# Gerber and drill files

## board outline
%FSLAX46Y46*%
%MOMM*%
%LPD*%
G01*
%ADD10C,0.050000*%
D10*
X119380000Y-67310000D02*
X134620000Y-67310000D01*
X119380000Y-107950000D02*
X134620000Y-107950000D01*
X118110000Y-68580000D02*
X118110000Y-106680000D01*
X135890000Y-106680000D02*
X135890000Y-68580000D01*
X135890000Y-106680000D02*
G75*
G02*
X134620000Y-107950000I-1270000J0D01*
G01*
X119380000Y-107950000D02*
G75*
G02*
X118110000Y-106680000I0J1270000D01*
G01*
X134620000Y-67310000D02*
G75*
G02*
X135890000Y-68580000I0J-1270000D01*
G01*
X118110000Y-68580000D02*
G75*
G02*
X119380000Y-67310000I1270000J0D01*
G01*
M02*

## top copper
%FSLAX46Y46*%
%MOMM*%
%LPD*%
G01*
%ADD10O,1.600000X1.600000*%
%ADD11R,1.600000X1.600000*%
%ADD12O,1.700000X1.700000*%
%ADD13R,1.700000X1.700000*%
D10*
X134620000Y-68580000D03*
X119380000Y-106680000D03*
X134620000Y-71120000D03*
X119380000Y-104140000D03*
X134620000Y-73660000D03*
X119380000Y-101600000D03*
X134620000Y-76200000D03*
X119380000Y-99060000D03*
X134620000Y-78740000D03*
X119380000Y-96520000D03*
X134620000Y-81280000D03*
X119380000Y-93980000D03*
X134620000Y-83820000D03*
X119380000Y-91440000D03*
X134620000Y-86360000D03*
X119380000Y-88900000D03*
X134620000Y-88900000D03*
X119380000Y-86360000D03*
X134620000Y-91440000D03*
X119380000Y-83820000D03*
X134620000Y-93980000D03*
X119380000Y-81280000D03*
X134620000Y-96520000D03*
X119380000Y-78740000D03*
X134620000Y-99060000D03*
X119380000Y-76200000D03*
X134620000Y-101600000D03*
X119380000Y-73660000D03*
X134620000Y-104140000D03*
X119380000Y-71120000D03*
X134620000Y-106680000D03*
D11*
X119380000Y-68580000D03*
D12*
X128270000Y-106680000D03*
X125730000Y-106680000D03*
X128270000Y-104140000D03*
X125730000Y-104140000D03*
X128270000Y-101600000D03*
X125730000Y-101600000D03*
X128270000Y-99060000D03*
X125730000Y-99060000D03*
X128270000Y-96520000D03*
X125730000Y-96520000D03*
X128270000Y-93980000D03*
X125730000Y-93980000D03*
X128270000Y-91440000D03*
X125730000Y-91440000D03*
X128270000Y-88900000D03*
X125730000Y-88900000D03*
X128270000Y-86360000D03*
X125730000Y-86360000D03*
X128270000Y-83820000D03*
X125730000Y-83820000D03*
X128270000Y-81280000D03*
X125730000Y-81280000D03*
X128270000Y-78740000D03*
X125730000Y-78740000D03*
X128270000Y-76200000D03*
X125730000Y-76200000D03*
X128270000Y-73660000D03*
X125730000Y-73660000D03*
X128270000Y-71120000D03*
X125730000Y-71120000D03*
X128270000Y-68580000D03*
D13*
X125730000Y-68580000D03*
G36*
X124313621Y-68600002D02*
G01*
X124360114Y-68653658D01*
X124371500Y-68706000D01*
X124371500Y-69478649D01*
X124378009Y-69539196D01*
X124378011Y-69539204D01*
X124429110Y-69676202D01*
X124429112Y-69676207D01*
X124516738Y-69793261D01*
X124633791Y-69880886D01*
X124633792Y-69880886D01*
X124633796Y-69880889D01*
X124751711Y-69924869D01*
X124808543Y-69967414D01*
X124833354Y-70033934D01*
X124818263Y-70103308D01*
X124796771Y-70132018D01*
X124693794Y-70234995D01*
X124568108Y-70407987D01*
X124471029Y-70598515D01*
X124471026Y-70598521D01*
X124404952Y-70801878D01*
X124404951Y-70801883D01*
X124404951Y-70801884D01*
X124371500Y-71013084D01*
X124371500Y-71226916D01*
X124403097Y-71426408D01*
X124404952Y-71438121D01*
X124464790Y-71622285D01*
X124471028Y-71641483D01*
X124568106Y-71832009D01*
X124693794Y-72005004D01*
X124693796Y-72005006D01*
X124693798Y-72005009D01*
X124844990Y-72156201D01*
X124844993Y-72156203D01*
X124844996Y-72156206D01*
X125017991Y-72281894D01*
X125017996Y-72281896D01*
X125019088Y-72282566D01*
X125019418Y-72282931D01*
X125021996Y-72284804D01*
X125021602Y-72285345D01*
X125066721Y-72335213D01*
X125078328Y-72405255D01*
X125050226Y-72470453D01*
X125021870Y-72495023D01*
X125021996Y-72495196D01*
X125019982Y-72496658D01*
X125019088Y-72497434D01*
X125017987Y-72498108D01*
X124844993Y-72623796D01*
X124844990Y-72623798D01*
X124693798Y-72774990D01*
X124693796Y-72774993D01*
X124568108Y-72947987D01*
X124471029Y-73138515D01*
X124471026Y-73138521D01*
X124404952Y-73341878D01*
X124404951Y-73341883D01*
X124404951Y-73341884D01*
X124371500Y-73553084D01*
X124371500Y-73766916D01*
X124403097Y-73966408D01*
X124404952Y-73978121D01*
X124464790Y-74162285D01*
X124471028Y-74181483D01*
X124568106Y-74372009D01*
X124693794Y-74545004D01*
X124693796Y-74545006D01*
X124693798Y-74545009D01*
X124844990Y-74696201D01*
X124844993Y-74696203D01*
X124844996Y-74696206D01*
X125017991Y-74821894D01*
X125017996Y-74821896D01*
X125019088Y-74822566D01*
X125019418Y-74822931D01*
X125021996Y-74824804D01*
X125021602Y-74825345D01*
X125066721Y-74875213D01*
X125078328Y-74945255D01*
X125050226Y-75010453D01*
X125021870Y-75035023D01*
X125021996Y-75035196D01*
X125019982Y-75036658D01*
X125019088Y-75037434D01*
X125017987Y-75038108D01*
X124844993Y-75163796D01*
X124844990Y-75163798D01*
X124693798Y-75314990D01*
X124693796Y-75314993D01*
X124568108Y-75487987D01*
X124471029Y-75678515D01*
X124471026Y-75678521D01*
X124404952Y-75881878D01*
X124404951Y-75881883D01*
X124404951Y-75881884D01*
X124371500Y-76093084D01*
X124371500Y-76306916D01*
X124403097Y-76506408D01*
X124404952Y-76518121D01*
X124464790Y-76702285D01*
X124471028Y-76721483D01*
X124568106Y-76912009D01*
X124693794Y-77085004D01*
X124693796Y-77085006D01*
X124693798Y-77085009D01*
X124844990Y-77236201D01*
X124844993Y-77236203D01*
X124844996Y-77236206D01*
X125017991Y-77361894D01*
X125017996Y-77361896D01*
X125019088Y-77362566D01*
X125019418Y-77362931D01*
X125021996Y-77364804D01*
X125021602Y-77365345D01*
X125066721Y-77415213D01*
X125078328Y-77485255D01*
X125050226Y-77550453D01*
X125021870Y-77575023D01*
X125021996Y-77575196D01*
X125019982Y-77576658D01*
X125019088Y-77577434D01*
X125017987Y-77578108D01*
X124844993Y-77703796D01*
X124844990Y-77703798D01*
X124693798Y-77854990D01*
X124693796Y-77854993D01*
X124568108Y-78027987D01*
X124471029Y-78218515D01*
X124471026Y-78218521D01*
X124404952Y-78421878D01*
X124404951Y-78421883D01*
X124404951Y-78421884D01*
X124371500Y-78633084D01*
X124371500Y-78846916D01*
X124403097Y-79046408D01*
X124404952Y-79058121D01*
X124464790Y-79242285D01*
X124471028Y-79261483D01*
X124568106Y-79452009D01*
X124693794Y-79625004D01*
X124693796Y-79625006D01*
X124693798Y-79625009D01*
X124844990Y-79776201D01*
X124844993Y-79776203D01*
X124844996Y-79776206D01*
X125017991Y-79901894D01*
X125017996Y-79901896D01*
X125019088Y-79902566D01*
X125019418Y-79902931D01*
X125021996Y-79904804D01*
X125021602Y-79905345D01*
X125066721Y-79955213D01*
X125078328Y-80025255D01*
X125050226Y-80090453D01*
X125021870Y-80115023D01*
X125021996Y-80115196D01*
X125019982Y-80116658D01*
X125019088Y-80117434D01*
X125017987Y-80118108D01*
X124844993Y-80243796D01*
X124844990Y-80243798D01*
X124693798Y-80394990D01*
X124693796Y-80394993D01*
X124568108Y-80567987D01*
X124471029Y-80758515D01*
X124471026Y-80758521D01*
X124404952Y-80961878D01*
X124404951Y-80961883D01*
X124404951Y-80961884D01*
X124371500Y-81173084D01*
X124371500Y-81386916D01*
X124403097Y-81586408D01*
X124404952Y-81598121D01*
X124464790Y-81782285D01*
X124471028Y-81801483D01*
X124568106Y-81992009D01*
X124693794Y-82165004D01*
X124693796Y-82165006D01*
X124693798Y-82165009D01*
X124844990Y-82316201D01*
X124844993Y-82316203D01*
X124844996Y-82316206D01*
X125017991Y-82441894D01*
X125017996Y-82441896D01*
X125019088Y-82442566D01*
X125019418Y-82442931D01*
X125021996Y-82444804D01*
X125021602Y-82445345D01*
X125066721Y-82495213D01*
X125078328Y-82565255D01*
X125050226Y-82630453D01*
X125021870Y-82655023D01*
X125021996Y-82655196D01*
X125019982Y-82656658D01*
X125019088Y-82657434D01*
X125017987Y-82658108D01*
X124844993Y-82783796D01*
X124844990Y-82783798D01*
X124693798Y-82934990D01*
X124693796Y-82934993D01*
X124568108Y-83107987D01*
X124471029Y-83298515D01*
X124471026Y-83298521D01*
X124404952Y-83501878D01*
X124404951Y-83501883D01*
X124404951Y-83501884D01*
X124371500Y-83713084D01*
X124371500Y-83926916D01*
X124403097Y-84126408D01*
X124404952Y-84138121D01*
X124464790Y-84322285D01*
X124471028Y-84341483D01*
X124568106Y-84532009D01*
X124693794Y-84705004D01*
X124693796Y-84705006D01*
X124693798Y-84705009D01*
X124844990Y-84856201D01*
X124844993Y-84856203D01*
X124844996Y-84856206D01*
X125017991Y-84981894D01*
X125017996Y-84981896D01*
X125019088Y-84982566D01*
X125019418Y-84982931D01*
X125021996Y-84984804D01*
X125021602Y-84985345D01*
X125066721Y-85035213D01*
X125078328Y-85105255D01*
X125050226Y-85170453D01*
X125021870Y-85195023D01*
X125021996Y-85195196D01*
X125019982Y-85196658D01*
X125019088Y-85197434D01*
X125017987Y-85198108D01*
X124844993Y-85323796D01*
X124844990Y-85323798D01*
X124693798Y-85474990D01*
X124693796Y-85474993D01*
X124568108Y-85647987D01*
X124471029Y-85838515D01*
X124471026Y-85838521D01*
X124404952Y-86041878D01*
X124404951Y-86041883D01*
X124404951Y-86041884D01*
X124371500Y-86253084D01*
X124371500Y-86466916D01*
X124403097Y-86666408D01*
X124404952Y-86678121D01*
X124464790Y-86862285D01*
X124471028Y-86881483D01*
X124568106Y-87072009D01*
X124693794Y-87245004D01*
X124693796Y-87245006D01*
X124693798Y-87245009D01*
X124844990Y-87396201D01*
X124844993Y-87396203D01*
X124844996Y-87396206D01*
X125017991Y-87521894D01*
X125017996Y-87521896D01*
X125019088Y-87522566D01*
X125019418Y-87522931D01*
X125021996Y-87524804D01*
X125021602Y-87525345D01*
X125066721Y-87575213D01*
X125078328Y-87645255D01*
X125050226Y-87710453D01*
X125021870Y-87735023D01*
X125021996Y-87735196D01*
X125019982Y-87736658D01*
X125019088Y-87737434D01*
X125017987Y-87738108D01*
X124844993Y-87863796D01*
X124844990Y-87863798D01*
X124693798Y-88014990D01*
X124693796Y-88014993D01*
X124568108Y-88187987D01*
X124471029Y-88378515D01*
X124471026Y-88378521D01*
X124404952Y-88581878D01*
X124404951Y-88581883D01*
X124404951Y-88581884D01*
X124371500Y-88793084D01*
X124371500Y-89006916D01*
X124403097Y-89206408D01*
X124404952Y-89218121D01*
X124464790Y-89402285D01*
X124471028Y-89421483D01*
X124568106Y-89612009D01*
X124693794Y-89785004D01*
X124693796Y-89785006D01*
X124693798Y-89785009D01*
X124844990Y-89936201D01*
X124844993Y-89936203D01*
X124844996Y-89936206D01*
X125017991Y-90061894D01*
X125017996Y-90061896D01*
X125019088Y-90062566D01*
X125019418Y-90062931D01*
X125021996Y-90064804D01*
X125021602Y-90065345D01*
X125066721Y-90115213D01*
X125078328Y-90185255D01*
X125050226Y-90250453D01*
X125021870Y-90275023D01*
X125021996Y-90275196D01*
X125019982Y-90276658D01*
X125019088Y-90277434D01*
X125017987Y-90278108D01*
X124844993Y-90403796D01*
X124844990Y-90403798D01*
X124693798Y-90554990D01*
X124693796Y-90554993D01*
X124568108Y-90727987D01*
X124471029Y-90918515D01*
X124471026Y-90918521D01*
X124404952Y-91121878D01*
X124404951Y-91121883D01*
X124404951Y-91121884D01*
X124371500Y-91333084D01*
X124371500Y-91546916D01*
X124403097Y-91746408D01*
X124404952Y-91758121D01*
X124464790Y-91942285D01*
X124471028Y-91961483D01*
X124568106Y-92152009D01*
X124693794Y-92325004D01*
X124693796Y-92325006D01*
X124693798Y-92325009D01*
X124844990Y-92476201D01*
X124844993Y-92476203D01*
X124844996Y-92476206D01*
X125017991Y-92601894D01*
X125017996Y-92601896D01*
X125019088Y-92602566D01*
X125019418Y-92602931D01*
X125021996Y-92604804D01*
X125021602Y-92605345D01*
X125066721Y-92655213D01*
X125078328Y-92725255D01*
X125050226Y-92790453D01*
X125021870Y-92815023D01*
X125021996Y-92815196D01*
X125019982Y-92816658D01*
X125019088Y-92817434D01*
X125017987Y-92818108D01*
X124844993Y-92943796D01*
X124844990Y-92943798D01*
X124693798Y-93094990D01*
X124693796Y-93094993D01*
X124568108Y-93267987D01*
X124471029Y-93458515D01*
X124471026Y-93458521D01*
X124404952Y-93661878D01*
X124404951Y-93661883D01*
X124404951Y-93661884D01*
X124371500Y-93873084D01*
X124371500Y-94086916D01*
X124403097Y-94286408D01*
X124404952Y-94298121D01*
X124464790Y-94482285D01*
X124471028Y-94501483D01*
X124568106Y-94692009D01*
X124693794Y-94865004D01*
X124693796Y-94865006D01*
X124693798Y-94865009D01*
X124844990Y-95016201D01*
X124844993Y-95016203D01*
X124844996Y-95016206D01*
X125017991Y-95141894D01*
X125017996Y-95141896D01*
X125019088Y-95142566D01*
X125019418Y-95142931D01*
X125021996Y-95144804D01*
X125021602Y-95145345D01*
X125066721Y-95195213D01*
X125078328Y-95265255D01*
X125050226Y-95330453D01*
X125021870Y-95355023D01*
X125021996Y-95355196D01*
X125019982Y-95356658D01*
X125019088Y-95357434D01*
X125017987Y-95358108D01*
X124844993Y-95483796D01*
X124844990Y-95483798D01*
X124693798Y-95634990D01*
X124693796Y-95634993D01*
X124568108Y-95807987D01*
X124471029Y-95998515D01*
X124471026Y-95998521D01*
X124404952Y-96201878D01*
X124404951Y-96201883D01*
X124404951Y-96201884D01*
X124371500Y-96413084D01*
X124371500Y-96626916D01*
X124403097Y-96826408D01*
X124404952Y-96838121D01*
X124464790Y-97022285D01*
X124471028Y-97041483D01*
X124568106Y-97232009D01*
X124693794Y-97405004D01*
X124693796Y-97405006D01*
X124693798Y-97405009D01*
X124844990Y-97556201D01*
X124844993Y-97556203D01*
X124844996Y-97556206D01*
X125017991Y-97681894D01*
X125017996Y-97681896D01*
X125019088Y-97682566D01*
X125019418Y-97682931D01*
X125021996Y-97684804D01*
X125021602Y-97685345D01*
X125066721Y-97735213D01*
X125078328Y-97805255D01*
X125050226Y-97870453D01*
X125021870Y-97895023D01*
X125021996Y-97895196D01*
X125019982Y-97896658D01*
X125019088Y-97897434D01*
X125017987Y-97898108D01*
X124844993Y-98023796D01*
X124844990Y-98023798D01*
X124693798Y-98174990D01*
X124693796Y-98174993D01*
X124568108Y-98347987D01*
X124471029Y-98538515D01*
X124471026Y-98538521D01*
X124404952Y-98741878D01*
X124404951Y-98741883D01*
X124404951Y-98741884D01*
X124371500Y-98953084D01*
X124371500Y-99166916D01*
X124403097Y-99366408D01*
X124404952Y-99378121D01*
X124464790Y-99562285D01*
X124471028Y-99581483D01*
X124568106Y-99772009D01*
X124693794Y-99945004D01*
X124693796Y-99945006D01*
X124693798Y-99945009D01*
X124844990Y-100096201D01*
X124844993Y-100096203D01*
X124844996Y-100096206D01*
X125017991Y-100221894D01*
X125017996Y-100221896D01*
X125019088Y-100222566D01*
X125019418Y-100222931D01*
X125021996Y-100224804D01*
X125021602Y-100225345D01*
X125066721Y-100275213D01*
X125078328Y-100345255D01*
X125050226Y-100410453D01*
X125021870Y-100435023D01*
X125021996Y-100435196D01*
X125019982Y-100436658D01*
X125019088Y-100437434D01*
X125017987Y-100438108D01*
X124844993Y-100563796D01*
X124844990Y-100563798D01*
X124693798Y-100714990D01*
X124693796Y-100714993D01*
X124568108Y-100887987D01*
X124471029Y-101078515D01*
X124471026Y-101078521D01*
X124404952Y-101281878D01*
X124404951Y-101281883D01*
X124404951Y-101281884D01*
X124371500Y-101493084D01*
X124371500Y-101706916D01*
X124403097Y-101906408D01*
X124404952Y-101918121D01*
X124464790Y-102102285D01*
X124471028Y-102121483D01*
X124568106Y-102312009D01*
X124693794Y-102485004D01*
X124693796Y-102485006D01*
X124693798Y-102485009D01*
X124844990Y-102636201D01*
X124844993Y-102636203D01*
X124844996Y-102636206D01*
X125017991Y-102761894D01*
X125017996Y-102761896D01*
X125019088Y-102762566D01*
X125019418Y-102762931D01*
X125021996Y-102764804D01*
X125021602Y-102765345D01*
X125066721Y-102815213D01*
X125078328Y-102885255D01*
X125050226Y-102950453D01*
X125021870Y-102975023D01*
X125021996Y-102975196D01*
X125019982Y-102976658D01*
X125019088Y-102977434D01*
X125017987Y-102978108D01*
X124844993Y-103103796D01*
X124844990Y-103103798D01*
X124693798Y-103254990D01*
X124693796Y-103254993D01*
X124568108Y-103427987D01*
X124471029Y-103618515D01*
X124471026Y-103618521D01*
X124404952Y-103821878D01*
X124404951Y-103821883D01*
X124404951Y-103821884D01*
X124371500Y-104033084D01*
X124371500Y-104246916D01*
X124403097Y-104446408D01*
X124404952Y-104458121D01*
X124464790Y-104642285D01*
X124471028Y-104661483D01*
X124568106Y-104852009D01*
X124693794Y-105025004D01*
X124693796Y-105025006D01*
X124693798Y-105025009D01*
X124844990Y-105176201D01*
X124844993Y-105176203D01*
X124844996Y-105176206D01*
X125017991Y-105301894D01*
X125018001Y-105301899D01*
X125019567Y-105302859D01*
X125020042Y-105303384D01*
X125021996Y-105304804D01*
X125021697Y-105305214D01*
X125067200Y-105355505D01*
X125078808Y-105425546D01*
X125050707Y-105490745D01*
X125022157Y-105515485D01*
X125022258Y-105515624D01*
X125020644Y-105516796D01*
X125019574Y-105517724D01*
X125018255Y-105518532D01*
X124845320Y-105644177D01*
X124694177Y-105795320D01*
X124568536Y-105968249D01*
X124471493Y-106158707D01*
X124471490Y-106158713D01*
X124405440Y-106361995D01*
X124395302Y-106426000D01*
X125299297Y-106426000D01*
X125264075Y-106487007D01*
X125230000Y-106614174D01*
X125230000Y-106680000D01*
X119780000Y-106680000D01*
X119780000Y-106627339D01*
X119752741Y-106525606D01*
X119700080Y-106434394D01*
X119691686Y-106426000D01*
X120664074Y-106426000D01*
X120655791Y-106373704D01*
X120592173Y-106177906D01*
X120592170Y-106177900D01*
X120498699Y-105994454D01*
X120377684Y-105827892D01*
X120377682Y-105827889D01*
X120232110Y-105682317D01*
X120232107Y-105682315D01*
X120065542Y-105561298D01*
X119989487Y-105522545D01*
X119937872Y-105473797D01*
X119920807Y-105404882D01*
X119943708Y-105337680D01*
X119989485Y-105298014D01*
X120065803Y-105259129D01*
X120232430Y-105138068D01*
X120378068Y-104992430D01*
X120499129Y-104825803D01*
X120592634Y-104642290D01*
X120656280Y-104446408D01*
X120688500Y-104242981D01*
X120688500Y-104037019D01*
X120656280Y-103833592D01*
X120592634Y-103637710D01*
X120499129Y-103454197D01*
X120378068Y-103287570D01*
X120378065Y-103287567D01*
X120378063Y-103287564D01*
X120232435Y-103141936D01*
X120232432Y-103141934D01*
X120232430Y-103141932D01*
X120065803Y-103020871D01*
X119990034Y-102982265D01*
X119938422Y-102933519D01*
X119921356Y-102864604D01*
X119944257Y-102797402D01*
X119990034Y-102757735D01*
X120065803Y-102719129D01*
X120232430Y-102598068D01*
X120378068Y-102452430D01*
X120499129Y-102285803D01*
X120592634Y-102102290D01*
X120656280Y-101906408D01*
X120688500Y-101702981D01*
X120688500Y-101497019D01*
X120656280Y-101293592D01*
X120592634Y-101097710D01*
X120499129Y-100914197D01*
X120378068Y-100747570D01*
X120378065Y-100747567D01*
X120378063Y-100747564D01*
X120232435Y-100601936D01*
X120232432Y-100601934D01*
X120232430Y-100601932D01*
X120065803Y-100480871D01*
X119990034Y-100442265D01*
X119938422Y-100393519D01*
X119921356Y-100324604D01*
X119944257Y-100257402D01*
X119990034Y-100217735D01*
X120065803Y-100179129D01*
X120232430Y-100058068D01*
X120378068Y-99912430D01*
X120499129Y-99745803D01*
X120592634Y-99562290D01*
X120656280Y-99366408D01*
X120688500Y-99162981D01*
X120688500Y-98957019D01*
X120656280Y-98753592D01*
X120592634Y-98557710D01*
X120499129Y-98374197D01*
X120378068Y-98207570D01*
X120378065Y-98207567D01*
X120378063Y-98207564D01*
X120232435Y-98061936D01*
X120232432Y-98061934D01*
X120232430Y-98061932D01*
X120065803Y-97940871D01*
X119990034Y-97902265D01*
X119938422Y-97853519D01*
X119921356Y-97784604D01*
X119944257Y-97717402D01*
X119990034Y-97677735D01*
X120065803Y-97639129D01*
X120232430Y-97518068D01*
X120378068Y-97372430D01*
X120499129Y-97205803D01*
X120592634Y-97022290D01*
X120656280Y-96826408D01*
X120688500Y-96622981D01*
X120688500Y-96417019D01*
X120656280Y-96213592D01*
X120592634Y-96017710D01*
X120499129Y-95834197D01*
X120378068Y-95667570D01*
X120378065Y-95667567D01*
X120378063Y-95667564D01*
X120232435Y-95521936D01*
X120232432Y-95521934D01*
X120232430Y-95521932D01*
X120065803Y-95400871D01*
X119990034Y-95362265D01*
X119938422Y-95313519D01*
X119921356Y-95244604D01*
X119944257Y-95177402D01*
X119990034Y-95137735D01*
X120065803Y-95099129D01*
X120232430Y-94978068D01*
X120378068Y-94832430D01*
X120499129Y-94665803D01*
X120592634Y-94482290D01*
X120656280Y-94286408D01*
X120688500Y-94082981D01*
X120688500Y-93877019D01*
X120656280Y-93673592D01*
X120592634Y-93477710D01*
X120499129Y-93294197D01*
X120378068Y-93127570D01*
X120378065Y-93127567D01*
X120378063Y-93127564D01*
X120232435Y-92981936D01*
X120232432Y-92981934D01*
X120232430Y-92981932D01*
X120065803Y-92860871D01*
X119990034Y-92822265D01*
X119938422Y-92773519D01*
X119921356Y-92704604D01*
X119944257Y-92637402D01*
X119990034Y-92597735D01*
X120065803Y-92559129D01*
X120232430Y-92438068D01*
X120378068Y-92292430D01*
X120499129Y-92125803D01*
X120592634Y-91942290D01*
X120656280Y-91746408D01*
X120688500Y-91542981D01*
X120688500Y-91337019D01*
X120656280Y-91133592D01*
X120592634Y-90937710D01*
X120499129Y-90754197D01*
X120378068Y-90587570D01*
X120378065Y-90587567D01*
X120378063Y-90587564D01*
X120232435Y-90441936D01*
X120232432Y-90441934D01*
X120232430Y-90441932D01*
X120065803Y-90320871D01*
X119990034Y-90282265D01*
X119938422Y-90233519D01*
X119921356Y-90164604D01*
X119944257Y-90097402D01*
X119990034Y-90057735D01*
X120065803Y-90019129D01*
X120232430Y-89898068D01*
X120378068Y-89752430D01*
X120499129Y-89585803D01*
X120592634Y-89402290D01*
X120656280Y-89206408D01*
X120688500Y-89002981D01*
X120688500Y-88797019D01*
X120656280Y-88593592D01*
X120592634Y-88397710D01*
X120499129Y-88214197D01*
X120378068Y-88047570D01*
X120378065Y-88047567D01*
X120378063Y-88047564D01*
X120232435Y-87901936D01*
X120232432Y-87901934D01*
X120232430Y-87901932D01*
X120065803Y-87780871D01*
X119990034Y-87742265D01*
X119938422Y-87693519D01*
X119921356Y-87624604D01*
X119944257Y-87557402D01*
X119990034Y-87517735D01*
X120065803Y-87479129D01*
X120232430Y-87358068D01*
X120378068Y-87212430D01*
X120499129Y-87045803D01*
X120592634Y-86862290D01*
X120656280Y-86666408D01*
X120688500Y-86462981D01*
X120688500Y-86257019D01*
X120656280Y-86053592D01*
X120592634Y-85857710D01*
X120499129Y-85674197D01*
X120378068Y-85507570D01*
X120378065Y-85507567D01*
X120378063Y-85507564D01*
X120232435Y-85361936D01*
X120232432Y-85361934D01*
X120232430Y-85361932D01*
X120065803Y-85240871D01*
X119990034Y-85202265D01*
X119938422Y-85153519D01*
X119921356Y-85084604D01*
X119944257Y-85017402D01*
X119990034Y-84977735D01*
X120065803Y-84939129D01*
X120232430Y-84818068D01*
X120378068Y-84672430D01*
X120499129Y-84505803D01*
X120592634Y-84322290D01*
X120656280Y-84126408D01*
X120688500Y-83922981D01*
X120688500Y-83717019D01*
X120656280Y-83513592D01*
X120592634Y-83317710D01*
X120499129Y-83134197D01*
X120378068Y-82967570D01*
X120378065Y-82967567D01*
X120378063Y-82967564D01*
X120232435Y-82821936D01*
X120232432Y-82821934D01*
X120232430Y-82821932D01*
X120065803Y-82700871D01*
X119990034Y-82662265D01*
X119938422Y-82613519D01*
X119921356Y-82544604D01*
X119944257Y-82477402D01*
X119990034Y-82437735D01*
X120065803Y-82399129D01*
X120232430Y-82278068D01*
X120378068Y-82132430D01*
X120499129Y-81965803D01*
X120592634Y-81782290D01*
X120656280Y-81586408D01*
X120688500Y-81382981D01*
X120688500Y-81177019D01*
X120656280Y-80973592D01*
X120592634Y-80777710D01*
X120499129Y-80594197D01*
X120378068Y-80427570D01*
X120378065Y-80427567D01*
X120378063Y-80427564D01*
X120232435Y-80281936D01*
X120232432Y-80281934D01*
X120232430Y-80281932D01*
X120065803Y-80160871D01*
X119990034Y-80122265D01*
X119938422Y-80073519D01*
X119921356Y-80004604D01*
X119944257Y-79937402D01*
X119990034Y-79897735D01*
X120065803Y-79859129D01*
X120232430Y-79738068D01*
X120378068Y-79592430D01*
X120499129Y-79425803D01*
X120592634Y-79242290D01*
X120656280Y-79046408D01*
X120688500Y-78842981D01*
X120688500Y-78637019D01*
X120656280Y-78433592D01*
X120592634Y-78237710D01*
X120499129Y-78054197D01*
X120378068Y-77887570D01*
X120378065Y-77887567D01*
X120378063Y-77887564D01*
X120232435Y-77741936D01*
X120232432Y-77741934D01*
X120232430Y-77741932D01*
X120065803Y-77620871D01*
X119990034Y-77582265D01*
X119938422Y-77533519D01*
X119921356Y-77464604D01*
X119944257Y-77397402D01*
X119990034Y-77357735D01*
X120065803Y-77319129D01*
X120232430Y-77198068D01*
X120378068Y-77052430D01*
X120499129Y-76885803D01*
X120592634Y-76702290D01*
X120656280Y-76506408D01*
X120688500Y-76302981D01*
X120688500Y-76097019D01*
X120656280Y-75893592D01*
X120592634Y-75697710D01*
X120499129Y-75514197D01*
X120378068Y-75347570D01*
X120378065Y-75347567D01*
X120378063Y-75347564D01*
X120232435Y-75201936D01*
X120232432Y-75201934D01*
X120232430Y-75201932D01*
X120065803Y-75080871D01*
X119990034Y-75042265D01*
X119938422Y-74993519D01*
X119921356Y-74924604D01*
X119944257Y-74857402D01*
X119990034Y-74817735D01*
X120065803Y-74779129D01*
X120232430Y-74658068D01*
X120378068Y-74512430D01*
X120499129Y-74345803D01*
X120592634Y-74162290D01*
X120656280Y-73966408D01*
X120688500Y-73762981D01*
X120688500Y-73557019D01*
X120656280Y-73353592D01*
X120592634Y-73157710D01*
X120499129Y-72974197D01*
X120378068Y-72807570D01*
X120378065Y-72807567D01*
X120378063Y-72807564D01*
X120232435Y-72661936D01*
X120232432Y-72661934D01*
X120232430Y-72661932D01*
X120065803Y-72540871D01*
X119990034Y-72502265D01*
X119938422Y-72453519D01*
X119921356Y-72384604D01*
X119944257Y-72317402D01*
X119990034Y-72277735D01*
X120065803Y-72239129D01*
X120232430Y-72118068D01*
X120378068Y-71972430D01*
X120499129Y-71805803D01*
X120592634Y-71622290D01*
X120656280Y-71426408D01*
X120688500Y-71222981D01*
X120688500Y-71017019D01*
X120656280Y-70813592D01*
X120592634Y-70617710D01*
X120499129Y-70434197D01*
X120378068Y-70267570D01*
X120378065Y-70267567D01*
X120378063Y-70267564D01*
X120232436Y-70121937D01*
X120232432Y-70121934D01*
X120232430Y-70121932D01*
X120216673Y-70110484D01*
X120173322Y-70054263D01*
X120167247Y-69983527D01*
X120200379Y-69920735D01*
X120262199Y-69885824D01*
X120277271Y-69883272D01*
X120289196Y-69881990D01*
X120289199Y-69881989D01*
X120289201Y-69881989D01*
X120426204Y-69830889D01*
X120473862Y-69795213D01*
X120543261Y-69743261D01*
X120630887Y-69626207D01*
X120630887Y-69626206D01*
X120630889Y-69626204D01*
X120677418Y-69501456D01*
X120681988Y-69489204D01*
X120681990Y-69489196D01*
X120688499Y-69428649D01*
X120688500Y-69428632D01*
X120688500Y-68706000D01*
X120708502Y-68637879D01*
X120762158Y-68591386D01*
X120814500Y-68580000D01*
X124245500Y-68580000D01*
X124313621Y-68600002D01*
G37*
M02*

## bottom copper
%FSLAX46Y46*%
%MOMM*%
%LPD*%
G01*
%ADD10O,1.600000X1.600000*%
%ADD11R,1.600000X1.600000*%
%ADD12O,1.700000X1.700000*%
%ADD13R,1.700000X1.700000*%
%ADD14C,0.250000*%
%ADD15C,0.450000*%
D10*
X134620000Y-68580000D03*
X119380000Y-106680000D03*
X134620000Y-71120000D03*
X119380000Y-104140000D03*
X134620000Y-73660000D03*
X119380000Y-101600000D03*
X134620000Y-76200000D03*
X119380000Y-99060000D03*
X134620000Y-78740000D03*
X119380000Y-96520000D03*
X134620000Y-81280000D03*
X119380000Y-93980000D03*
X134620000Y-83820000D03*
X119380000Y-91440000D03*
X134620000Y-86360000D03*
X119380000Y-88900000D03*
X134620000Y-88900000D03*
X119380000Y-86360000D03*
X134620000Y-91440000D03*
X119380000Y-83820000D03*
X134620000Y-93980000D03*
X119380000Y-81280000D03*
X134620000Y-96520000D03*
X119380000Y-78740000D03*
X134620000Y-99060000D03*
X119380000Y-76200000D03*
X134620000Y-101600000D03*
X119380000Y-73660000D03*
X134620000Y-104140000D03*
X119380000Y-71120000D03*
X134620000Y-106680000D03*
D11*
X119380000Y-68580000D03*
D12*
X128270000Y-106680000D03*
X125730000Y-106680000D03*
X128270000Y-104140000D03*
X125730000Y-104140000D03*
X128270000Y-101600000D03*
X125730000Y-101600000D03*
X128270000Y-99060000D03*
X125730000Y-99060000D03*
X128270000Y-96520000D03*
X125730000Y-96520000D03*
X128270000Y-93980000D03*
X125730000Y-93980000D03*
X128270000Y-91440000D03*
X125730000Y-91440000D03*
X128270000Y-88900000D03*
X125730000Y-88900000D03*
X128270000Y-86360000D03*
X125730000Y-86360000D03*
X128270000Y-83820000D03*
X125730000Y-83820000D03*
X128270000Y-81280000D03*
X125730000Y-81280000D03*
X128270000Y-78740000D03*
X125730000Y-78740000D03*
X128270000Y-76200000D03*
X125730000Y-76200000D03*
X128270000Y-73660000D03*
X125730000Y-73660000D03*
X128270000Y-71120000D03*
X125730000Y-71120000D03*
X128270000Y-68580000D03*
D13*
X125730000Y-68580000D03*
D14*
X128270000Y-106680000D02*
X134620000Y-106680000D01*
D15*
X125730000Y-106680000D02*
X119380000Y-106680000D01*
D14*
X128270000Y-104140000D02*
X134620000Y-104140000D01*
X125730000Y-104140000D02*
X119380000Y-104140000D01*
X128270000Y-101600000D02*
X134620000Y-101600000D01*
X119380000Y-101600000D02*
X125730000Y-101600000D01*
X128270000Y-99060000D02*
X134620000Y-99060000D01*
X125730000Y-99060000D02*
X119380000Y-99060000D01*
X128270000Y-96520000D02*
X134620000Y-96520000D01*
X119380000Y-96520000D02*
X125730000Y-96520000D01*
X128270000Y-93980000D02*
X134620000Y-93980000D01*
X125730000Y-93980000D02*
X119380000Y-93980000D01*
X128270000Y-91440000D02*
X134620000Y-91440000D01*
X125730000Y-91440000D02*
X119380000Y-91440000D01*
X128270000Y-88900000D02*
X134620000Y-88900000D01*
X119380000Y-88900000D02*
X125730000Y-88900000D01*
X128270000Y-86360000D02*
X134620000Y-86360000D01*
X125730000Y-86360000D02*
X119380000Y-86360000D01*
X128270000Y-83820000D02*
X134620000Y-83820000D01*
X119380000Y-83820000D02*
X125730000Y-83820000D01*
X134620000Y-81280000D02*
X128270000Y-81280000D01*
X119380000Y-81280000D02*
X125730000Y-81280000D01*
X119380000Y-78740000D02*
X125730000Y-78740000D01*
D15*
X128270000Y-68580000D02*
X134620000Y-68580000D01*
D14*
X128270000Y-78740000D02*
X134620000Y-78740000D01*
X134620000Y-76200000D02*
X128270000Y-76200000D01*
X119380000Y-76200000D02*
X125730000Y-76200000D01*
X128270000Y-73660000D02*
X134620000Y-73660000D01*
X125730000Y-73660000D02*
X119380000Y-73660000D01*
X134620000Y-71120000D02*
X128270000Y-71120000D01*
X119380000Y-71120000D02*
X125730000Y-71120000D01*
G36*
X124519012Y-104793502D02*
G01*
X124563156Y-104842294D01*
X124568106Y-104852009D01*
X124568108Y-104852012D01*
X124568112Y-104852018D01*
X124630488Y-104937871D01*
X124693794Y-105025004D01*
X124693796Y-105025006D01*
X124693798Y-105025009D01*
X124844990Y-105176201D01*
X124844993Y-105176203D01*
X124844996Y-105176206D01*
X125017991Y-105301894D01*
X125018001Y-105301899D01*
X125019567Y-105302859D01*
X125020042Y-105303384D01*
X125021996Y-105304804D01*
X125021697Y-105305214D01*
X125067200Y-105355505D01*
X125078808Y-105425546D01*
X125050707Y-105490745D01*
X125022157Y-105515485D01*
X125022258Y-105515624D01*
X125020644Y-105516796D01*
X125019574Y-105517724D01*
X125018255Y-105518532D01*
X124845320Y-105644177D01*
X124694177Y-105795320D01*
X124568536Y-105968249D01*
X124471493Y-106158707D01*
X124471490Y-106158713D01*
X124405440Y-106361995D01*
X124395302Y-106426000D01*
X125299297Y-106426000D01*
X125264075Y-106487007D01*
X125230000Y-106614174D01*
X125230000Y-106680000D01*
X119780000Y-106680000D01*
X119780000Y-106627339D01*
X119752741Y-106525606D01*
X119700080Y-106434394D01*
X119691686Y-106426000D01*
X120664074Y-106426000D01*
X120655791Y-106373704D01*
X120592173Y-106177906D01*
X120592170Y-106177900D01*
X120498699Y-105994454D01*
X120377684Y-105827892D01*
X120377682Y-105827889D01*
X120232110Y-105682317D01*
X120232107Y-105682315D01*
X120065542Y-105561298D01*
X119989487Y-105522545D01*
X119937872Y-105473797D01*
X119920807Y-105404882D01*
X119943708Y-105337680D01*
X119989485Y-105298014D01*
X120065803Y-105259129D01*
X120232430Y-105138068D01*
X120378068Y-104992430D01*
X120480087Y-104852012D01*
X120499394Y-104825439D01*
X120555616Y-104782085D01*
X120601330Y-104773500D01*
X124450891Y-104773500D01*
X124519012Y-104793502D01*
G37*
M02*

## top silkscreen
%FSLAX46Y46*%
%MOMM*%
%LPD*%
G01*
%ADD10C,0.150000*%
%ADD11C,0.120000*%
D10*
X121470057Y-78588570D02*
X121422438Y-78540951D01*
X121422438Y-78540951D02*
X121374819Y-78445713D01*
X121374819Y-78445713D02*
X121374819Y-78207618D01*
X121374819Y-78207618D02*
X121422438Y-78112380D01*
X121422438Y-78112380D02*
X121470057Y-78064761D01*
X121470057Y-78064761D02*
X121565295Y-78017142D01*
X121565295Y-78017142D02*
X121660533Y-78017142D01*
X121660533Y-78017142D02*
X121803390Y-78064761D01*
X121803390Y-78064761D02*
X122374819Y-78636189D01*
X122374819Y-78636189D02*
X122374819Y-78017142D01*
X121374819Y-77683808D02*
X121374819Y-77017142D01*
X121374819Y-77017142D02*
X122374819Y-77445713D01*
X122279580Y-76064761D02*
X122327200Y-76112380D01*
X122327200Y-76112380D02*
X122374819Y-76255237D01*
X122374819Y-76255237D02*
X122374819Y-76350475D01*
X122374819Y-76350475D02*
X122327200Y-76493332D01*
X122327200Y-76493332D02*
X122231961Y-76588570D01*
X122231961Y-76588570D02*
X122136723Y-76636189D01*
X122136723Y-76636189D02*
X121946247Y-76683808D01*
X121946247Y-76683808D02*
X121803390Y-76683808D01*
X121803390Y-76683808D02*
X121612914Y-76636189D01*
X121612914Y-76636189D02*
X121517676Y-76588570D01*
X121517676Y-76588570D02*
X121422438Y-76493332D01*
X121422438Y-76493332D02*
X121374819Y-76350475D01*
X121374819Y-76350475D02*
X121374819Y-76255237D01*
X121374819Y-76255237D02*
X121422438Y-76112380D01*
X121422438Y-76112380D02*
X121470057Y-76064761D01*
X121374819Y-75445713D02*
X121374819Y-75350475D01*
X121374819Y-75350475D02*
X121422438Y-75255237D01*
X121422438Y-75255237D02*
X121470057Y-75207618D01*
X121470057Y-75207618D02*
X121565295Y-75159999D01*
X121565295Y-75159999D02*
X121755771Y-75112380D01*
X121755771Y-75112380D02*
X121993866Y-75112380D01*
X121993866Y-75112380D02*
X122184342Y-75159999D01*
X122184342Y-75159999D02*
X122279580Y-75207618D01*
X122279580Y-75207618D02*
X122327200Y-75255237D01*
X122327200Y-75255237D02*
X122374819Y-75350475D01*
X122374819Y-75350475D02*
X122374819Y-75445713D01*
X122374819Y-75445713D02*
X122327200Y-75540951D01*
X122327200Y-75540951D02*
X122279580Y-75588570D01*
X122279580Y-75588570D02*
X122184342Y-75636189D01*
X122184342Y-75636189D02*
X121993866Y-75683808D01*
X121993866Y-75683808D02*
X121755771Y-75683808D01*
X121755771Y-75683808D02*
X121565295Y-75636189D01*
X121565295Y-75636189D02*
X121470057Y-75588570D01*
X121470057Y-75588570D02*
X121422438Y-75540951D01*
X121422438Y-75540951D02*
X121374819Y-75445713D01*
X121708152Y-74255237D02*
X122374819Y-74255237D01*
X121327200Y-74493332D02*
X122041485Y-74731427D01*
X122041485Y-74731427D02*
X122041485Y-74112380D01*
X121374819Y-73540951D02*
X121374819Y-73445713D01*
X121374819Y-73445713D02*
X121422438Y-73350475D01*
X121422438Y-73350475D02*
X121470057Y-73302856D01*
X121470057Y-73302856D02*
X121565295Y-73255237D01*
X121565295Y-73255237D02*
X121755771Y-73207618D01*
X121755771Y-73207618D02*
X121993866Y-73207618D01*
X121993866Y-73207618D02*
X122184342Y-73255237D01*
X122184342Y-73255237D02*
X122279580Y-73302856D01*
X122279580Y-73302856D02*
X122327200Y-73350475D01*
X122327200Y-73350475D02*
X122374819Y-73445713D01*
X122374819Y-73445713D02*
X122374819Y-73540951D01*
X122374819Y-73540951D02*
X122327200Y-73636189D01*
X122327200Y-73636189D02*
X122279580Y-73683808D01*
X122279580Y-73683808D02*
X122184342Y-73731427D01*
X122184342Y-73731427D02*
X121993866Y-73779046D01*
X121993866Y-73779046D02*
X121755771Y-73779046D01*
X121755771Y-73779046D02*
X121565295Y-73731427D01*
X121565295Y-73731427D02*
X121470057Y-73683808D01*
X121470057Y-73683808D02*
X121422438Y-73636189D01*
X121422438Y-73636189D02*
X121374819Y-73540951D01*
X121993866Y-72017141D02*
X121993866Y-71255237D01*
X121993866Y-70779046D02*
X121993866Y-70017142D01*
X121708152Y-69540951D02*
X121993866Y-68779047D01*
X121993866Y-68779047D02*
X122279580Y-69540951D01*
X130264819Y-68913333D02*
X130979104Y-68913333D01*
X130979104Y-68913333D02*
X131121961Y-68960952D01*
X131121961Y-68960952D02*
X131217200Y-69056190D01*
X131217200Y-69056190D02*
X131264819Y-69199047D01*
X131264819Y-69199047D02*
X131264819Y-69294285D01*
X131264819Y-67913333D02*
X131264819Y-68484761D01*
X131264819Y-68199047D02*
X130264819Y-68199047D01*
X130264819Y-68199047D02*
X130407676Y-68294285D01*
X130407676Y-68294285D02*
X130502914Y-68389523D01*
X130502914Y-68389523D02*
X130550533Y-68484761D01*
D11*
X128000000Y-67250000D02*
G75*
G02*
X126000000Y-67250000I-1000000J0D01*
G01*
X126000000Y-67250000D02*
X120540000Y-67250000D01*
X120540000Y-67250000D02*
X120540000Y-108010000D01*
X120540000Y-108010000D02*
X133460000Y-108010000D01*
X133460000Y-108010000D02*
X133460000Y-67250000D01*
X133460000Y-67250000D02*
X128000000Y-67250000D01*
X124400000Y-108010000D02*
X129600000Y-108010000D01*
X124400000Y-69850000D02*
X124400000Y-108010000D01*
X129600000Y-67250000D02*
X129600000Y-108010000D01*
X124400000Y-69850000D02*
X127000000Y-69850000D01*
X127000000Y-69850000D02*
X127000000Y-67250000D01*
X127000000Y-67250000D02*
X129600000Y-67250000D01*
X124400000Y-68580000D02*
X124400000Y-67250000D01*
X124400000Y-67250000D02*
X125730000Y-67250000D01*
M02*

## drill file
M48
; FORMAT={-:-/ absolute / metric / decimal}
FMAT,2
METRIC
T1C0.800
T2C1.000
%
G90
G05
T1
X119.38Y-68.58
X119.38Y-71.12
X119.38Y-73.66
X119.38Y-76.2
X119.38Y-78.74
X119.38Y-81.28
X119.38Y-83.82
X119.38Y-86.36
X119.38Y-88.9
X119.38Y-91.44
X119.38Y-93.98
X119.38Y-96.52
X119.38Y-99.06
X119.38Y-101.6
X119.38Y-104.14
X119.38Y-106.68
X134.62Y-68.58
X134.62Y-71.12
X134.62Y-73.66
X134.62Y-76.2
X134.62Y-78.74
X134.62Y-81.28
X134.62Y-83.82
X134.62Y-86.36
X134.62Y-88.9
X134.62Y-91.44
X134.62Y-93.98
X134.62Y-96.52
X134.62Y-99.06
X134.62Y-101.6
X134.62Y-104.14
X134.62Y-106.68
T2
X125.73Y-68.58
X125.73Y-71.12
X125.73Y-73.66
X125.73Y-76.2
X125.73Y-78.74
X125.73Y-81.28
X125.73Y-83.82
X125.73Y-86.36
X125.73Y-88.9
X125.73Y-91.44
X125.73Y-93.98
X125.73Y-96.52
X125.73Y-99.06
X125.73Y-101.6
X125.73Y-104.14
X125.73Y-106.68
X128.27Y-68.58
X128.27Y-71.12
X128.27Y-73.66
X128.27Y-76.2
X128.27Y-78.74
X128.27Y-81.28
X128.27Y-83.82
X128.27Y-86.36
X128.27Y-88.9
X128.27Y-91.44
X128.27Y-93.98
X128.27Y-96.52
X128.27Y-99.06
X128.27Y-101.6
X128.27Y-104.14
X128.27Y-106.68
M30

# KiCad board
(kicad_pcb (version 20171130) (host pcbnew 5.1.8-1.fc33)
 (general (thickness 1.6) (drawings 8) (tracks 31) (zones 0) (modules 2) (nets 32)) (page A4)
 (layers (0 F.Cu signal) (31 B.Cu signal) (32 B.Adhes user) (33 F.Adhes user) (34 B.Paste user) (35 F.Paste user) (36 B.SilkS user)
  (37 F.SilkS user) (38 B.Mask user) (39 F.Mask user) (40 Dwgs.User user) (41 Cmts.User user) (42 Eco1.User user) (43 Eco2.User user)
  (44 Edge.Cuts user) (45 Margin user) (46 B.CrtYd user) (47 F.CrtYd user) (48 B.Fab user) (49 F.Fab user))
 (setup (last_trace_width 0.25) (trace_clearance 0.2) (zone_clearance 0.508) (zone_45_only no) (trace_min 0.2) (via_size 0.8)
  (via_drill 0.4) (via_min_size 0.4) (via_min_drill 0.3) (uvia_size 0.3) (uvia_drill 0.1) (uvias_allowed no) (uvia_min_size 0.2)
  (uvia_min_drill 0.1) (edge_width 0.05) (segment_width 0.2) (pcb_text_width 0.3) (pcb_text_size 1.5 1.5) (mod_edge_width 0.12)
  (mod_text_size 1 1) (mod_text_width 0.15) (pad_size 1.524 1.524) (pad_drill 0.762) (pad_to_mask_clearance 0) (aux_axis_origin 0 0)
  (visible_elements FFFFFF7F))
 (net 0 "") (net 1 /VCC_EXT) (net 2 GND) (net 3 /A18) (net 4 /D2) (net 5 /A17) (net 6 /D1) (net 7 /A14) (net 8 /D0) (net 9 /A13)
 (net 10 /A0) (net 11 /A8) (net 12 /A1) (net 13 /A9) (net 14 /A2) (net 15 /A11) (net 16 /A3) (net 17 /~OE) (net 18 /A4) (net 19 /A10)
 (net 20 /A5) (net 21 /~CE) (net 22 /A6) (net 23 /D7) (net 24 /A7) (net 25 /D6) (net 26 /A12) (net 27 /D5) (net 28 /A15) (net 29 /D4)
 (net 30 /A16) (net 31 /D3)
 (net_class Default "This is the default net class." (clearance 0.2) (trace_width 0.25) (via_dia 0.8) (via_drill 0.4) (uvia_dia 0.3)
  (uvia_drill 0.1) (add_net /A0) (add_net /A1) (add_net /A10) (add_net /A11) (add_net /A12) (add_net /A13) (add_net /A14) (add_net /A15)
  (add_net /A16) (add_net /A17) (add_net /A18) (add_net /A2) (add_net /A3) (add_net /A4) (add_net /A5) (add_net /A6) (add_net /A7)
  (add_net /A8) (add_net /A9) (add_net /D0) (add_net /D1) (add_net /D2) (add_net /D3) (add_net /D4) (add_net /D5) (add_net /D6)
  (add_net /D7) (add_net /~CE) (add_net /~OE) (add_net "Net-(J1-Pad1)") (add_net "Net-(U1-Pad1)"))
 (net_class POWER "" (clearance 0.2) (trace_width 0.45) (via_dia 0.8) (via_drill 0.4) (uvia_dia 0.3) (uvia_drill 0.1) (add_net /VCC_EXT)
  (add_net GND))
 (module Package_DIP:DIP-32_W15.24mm (layer F.Cu) (at 119.38 68.58)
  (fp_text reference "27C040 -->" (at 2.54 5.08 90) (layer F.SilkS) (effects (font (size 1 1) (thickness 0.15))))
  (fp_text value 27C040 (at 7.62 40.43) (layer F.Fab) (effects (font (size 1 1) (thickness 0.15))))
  (fp_arc (start 7.62 -1.33) (end 6.62 -1.33) (angle -180) (layer F.SilkS) (width 0.12))
  (fp_line (start 6.62 -1.33) (end 1.16 -1.33) (layer F.SilkS) (width 0.12))
  (fp_line (start 1.16 -1.33) (end 1.16 39.43) (layer F.SilkS) (width 0.12))
  (fp_line (start 1.16 39.43) (end 14.08 39.43) (layer F.SilkS) (width 0.12))
  (fp_line (start 14.08 39.43) (end 14.08 -1.33) (layer F.SilkS) (width 0.12))
  (fp_line (start 14.08 -1.33) (end 8.62 -1.33) (layer F.SilkS) (width 0.12))
  (pad 32 thru_hole oval (at 15.24 0) (size 1.6 1.6) (drill 0.8) (layers *.Cu *.Mask) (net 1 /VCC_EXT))
  (pad 16 thru_hole oval (at 0 38.1) (size 1.6 1.6) (drill 0.8) (layers *.Cu *.Mask) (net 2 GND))
  (pad 31 thru_hole oval (at 15.24 2.54) (size 1.6 1.6) (drill 0.8) (layers *.Cu *.Mask) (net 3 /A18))
  (pad 15 thru_hole oval (at 0 35.56) (size 1.6 1.6) (drill 0.8) (layers *.Cu *.Mask) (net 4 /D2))
  (pad 30 thru_hole oval (at 15.24 5.08) (size 1.6 1.6) (drill 0.8) (layers *.Cu *.Mask) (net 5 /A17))
  (pad 14 thru_hole oval (at 0 33.02) (size 1.6 1.6) (drill 0.8) (layers *.Cu *.Mask) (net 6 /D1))
  (pad 29 thru_hole oval (at 15.24 7.62) (size 1.6 1.6) (drill 0.8) (layers *.Cu *.Mask) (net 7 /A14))
  (pad 13 thru_hole oval (at 0 30.48) (size 1.6 1.6) (drill 0.8) (layers *.Cu *.Mask) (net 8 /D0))
  (pad 28 thru_hole oval (at 15.24 10.16) (size 1.6 1.6) (drill 0.8) (layers *.Cu *.Mask) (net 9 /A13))
  (pad 12 thru_hole oval (at 0 27.94) (size 1.6 1.6) (drill 0.8) (layers *.Cu *.Mask) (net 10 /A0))
  (pad 27 thru_hole oval (at 15.24 12.7) (size 1.6 1.6) (drill 0.8) (layers *.Cu *.Mask) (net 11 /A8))
  (pad 11 thru_hole oval (at 0 25.4) (size 1.6 1.6) (drill 0.8) (layers *.Cu *.Mask) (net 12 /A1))
  (pad 26 thru_hole oval (at 15.24 15.24) (size 1.6 1.6) (drill 0.8) (layers *.Cu *.Mask) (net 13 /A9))
  (pad 10 thru_hole oval (at 0 22.86) (size 1.6 1.6) (drill 0.8) (layers *.Cu *.Mask) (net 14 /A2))
  (pad 25 thru_hole oval (at 15.24 17.78) (size 1.6 1.6) (drill 0.8) (layers *.Cu *.Mask) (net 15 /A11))
  (pad 9 thru_hole oval (at 0 20.32) (size 1.6 1.6) (drill 0.8) (layers *.Cu *.Mask) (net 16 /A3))
  (pad 24 thru_hole oval (at 15.24 20.32) (size 1.6 1.6) (drill 0.8) (layers *.Cu *.Mask) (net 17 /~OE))
  (pad 8 thru_hole oval (at 0 17.78) (size 1.6 1.6) (drill 0.8) (layers *.Cu *.Mask) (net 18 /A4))
  (pad 23 thru_hole oval (at 15.24 22.86) (size 1.6 1.6) (drill 0.8) (layers *.Cu *.Mask) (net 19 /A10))
  (pad 7 thru_hole oval (at 0 15.24) (size 1.6 1.6) (drill 0.8) (layers *.Cu *.Mask) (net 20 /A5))
  (pad 22 thru_hole oval (at 15.24 25.4) (size 1.6 1.6) (drill 0.8) (layers *.Cu *.Mask) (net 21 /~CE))
  (pad 6 thru_hole oval (at 0 12.7) (size 1.6 1.6) (drill 0.8) (layers *.Cu *.Mask) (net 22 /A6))
  (pad 21 thru_hole oval (at 15.24 27.94) (size 1.6 1.6) (drill 0.8) (layers *.Cu *.Mask) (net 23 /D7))
  (pad 5 thru_hole oval (at 0 10.16) (size 1.6 1.6) (drill 0.8) (layers *.Cu *.Mask) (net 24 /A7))
  (pad 20 thru_hole oval (at 15.24 30.48) (size 1.6 1.6) (drill 0.8) (layers *.Cu *.Mask) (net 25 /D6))
  (pad 4 thru_hole oval (at 0 7.62) (size 1.6 1.6) (drill 0.8) (layers *.Cu *.Mask) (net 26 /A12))
  (pad 19 thru_hole oval (at 15.24 33.02) (size 1.6 1.6) (drill 0.8) (layers *.Cu *.Mask) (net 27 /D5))
  (pad 3 thru_hole oval (at 0 5.08) (size 1.6 1.6) (drill 0.8) (layers *.Cu *.Mask) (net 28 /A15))
  (pad 18 thru_hole oval (at 15.24 35.56) (size 1.6 1.6) (drill 0.8) (layers *.Cu *.Mask) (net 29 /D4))
  (pad 2 thru_hole oval (at 0 2.54) (size 1.6 1.6) (drill 0.8) (layers *.Cu *.Mask) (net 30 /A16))
  (pad 17 thru_hole oval (at 15.24 38.1) (size 1.6 1.6) (drill 0.8) (layers *.Cu *.Mask) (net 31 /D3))
  (pad 1 thru_hole rect (at 0 0) (size 1.6 1.6) (drill 0.8) (layers *.Cu *.Mask)))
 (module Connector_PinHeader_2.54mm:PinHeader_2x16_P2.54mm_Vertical (layer F.Cu) (at 125.73 68.58)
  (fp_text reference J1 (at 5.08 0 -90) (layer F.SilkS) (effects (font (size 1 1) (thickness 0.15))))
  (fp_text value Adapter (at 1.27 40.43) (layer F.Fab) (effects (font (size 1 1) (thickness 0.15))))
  (fp_line (start -1.33 39.43) (end 3.87 39.43) (layer F.SilkS) (width 0.12))
  (fp_line (start -1.33 1.27) (end -1.33 39.43) (layer F.SilkS) (width 0.12))
  (fp_line (start 3.87 -1.33) (end 3.87 39.43) (layer F.SilkS) (width 0.12))
  (fp_line (start -1.33 1.27) (end 1.27 1.27) (layer F.SilkS) (width 0.12))
  (fp_line (start 1.27 1.27) (end 1.27 -1.33) (layer F.SilkS) (width 0.12))
  (fp_line (start 1.27 -1.33) (end 3.87 -1.33) (layer F.SilkS) (width 0.12))
  (fp_line (start -1.33 0) (end -1.33 -1.33) (layer F.SilkS) (width 0.12))
  (fp_line (start -1.33 -1.33) (end 0 -1.33) (layer F.SilkS) (width 0.12))
  (pad 32 thru_hole oval (at 2.54 38.1) (size 1.7 1.7) (drill 1) (layers *.Cu *.Mask) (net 31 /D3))
  (pad 31 thru_hole oval (at 0 38.1) (size 1.7 1.7) (drill 1) (layers *.Cu *.Mask) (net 2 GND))
  (pad 30 thru_hole oval (at 2.54 35.56) (size 1.7 1.7) (drill 1) (layers *.Cu *.Mask) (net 29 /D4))
  (pad 29 thru_hole oval (at 0 35.56) (size 1.7 1.7) (drill 1) (layers *.Cu *.Mask) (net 4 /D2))
  (pad 28 thru_hole oval (at 2.54 33.02) (size 1.7 1.7) (drill 1) (layers *.Cu *.Mask) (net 27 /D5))
  (pad 27 thru_hole oval (at 0 33.02) (size 1.7 1.7) (drill 1) (layers *.Cu *.Mask) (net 6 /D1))
  (pad 26 thru_hole oval (at 2.54 30.48) (size 1.7 1.7) (drill 1) (layers *.Cu *.Mask) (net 25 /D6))
  (pad 25 thru_hole oval (at 0 30.48) (size 1.7 1.7) (drill 1) (layers *.Cu *.Mask) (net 8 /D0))
  (pad 24 thru_hole oval (at 2.54 27.94) (size 1.7 1.7) (drill 1) (layers *.Cu *.Mask) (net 23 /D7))
  (pad 23 thru_hole oval (at 0 27.94) (size 1.7 1.7) (drill 1) (layers *.Cu *.Mask) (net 10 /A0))
  (pad 22 thru_hole oval (at 2.54 25.4) (size 1.7 1.7) (drill 1) (layers *.Cu *.Mask) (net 21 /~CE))
  (pad 21 thru_hole oval (at 0 25.4) (size 1.7 1.7) (drill 1) (layers *.Cu *.Mask) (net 12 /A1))
  (pad 20 thru_hole oval (at 2.54 22.86) (size 1.7 1.7) (drill 1) (layers *.Cu *.Mask) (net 19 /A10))
  (pad 19 thru_hole oval (at 0 22.86) (size 1.7 1.7) (drill 1) (layers *.Cu *.Mask) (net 14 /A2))
  (pad 18 thru_hole oval (at 2.54 20.32) (size 1.7 1.7) (drill 1) (layers *.Cu *.Mask) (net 17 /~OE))
  (pad 17 thru_hole oval (at 0 20.32) (size 1.7 1.7) (drill 1) (layers *.Cu *.Mask) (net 16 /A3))
  (pad 16 thru_hole oval (at 2.54 17.78) (size 1.7 1.7) (drill 1) (layers *.Cu *.Mask) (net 15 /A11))
  (pad 15 thru_hole oval (at 0 17.78) (size 1.7 1.7) (drill 1) (layers *.Cu *.Mask) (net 18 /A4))
  (pad 14 thru_hole oval (at 2.54 15.24) (size 1.7 1.7) (drill 1) (layers *.Cu *.Mask) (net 13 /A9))
  (pad 13 thru_hole oval (at 0 15.24) (size 1.7 1.7) (drill 1) (layers *.Cu *.Mask) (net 20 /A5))
  (pad 12 thru_hole oval (at 2.54 12.7) (size 1.7 1.7) (drill 1) (layers *.Cu *.Mask) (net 11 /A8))
  (pad 11 thru_hole oval (at 0 12.7) (size 1.7 1.7) (drill 1) (layers *.Cu *.Mask) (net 22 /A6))
  (pad 10 thru_hole oval (at 2.54 10.16) (size 1.7 1.7) (drill 1) (layers *.Cu *.Mask) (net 9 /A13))
  (pad 9 thru_hole oval (at 0 10.16) (size 1.7 1.7) (drill 1) (layers *.Cu *.Mask) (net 24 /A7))
  (pad 8 thru_hole oval (at 2.54 7.62) (size 1.7 1.7) (drill 1) (layers *.Cu *.Mask) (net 7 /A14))
  (pad 7 thru_hole oval (at 0 7.62) (size 1.7 1.7) (drill 1) (layers *.Cu *.Mask) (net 26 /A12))
  (pad 6 thru_hole oval (at 2.54 5.08) (size 1.7 1.7) (drill 1) (layers *.Cu *.Mask) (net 5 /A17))
  (pad 5 thru_hole oval (at 0 5.08) (size 1.7 1.7) (drill 1) (layers *.Cu *.Mask) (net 28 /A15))
  (pad 4 thru_hole oval (at 2.54 2.54) (size 1.7 1.7) (drill 1) (layers *.Cu *.Mask) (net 3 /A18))
  (pad 3 thru_hole oval (at 0 2.54) (size 1.7 1.7) (drill 1) (layers *.Cu *.Mask) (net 30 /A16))
  (pad 2 thru_hole oval (at 2.54 0) (size 1.7 1.7) (drill 1) (layers *.Cu *.Mask) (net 1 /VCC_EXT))
  (pad 1 thru_hole rect (at 0 0) (size 1.7 1.7) (drill 1) (layers *.Cu *.Mask)))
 (gr_line (start 119.38 67.31) (end 134.62 67.31) (layer Edge.Cuts) (width 0.05))
 (gr_line (start 119.38 107.95) (end 134.62 107.95) (layer Edge.Cuts) (width 0.05))
 (gr_line (start 118.11 68.58) (end 118.11 106.68) (layer Edge.Cuts) (width 0.05))
 (gr_line (start 135.89 106.68) (end 135.89 68.58) (layer Edge.Cuts) (width 0.05))
 (gr_arc (start 134.62 106.68) (end 134.62 107.95) (angle -90) (layer Edge.Cuts) (width 0.05))
 (gr_arc (start 119.38 106.68) (end 118.11 106.68) (angle -90) (layer Edge.Cuts) (width 0.05))
 (gr_arc (start 134.62 68.58) (end 135.89 68.58) (angle -90) (layer Edge.Cuts) (width 0.05))
 (gr_arc (start 119.38 68.58) (end 119.38 67.31) (angle -90) (layer Edge.Cuts) (width 0.05))
 (segment (start 128.27 106.68) (end 134.62 106.68) (width 0.25) (layer B.Cu) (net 31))
 (segment (start 125.73 106.68) (end 119.38 106.68) (width 0.45) (layer B.Cu) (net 2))
 (segment (start 128.27 104.14) (end 134.62 104.14) (width 0.25) (layer B.Cu) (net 29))
 (segment (start 125.73 104.14) (end 119.38 104.14) (width 0.25) (layer B.Cu) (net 4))
 (segment (start 128.27 101.6) (end 134.62 101.6) (width 0.25) (layer B.Cu) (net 27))
 (segment (start 119.38 101.6) (end 125.73 101.6) (width 0.25) (layer B.Cu) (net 6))
 (segment (start 128.27 99.06) (end 134.62 99.06) (width 0.25) (layer B.Cu) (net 25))
 (segment (start 125.73 99.06) (end 119.38 99.06) (width 0.25) (layer B.Cu) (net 8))
 (segment (start 128.27 96.52) (end 134.62 96.52) (width 0.25) (layer B.Cu) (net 23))
 (segment (start 119.38 96.52) (end 125.73 96.52) (width 0.25) (layer B.Cu) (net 10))
 (segment (start 128.27 93.98) (end 134.62 93.98) (width 0.25) (layer B.Cu) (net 21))
 (segment (start 125.73 93.98) (end 119.38 93.98) (width 0.25) (layer B.Cu) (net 12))
 (segment (start 128.27 91.44) (end 134.62 91.44) (width 0.25) (layer B.Cu) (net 19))
 (segment (start 125.73 91.44) (end 119.38 91.44) (width 0.25) (layer B.Cu) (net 14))
 (segment (start 128.27 88.9) (end 134.62 88.9) (width 0.25) (layer B.Cu) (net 17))
 (segment (start 119.38 88.9) (end 125.73 88.9) (width 0.25) (layer B.Cu) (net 16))
 (segment (start 128.27 86.36) (end 134.62 86.36) (width 0.25) (layer B.Cu) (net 15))
 (segment (start 125.73 86.36) (end 119.38 86.36) (width 0.25) (layer B.Cu) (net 18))
 (segment (start 128.27 83.82) (end 134.62 83.82) (width 0.25) (layer B.Cu) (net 13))
 (segment (start 119.38 83.82) (end 125.73 83.82) (width 0.25) (layer B.Cu) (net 20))
 (segment (start 134.62 81.28) (end 128.27 81.28) (width 0.25) (layer B.Cu) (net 11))
 (segment (start 119.38 81.28) (end 125.73 81.28) (width 0.25) (layer B.Cu) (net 22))
 (segment (start 119.38 78.74) (end 125.73 78.74) (width 0.25) (layer B.Cu) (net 24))
 (segment (start 128.27 68.58) (end 134.62 68.58) (width 0.45) (layer B.Cu) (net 1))
 (segment (start 128.27 78.74) (end 134.62 78.74) (width 0.25) (layer B.Cu) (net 9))
 (segment (start 134.62 76.2) (end 128.27 76.2) (width 0.25) (layer B.Cu) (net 7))
 (segment (start 119.38 76.2) (end 125.73 76.2) (width 0.25) (layer B.Cu) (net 26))
 (segment (start 128.27 73.66) (end 134.62 73.66) (width 0.25) (layer B.Cu) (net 5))
 (segment (start 125.73 73.66) (end 119.38 73.66) (width 0.25) (layer B.Cu) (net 28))
 (segment (start 134.62 71.12) (end 128.27 71.12) (width 0.25) (layer B.Cu) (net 3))
 (segment (start 119.38 71.12) (end 125.73 71.12) (width 0.25) (layer B.Cu) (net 30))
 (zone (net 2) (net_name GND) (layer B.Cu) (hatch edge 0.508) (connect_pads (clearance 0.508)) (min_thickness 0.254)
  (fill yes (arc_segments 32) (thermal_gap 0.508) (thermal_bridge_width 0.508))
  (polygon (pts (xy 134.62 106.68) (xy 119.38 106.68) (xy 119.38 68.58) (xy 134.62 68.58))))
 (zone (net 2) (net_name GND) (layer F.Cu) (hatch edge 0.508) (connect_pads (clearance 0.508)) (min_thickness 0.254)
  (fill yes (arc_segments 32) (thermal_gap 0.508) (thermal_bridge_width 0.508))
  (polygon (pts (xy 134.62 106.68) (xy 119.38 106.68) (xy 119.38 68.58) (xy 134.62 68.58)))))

